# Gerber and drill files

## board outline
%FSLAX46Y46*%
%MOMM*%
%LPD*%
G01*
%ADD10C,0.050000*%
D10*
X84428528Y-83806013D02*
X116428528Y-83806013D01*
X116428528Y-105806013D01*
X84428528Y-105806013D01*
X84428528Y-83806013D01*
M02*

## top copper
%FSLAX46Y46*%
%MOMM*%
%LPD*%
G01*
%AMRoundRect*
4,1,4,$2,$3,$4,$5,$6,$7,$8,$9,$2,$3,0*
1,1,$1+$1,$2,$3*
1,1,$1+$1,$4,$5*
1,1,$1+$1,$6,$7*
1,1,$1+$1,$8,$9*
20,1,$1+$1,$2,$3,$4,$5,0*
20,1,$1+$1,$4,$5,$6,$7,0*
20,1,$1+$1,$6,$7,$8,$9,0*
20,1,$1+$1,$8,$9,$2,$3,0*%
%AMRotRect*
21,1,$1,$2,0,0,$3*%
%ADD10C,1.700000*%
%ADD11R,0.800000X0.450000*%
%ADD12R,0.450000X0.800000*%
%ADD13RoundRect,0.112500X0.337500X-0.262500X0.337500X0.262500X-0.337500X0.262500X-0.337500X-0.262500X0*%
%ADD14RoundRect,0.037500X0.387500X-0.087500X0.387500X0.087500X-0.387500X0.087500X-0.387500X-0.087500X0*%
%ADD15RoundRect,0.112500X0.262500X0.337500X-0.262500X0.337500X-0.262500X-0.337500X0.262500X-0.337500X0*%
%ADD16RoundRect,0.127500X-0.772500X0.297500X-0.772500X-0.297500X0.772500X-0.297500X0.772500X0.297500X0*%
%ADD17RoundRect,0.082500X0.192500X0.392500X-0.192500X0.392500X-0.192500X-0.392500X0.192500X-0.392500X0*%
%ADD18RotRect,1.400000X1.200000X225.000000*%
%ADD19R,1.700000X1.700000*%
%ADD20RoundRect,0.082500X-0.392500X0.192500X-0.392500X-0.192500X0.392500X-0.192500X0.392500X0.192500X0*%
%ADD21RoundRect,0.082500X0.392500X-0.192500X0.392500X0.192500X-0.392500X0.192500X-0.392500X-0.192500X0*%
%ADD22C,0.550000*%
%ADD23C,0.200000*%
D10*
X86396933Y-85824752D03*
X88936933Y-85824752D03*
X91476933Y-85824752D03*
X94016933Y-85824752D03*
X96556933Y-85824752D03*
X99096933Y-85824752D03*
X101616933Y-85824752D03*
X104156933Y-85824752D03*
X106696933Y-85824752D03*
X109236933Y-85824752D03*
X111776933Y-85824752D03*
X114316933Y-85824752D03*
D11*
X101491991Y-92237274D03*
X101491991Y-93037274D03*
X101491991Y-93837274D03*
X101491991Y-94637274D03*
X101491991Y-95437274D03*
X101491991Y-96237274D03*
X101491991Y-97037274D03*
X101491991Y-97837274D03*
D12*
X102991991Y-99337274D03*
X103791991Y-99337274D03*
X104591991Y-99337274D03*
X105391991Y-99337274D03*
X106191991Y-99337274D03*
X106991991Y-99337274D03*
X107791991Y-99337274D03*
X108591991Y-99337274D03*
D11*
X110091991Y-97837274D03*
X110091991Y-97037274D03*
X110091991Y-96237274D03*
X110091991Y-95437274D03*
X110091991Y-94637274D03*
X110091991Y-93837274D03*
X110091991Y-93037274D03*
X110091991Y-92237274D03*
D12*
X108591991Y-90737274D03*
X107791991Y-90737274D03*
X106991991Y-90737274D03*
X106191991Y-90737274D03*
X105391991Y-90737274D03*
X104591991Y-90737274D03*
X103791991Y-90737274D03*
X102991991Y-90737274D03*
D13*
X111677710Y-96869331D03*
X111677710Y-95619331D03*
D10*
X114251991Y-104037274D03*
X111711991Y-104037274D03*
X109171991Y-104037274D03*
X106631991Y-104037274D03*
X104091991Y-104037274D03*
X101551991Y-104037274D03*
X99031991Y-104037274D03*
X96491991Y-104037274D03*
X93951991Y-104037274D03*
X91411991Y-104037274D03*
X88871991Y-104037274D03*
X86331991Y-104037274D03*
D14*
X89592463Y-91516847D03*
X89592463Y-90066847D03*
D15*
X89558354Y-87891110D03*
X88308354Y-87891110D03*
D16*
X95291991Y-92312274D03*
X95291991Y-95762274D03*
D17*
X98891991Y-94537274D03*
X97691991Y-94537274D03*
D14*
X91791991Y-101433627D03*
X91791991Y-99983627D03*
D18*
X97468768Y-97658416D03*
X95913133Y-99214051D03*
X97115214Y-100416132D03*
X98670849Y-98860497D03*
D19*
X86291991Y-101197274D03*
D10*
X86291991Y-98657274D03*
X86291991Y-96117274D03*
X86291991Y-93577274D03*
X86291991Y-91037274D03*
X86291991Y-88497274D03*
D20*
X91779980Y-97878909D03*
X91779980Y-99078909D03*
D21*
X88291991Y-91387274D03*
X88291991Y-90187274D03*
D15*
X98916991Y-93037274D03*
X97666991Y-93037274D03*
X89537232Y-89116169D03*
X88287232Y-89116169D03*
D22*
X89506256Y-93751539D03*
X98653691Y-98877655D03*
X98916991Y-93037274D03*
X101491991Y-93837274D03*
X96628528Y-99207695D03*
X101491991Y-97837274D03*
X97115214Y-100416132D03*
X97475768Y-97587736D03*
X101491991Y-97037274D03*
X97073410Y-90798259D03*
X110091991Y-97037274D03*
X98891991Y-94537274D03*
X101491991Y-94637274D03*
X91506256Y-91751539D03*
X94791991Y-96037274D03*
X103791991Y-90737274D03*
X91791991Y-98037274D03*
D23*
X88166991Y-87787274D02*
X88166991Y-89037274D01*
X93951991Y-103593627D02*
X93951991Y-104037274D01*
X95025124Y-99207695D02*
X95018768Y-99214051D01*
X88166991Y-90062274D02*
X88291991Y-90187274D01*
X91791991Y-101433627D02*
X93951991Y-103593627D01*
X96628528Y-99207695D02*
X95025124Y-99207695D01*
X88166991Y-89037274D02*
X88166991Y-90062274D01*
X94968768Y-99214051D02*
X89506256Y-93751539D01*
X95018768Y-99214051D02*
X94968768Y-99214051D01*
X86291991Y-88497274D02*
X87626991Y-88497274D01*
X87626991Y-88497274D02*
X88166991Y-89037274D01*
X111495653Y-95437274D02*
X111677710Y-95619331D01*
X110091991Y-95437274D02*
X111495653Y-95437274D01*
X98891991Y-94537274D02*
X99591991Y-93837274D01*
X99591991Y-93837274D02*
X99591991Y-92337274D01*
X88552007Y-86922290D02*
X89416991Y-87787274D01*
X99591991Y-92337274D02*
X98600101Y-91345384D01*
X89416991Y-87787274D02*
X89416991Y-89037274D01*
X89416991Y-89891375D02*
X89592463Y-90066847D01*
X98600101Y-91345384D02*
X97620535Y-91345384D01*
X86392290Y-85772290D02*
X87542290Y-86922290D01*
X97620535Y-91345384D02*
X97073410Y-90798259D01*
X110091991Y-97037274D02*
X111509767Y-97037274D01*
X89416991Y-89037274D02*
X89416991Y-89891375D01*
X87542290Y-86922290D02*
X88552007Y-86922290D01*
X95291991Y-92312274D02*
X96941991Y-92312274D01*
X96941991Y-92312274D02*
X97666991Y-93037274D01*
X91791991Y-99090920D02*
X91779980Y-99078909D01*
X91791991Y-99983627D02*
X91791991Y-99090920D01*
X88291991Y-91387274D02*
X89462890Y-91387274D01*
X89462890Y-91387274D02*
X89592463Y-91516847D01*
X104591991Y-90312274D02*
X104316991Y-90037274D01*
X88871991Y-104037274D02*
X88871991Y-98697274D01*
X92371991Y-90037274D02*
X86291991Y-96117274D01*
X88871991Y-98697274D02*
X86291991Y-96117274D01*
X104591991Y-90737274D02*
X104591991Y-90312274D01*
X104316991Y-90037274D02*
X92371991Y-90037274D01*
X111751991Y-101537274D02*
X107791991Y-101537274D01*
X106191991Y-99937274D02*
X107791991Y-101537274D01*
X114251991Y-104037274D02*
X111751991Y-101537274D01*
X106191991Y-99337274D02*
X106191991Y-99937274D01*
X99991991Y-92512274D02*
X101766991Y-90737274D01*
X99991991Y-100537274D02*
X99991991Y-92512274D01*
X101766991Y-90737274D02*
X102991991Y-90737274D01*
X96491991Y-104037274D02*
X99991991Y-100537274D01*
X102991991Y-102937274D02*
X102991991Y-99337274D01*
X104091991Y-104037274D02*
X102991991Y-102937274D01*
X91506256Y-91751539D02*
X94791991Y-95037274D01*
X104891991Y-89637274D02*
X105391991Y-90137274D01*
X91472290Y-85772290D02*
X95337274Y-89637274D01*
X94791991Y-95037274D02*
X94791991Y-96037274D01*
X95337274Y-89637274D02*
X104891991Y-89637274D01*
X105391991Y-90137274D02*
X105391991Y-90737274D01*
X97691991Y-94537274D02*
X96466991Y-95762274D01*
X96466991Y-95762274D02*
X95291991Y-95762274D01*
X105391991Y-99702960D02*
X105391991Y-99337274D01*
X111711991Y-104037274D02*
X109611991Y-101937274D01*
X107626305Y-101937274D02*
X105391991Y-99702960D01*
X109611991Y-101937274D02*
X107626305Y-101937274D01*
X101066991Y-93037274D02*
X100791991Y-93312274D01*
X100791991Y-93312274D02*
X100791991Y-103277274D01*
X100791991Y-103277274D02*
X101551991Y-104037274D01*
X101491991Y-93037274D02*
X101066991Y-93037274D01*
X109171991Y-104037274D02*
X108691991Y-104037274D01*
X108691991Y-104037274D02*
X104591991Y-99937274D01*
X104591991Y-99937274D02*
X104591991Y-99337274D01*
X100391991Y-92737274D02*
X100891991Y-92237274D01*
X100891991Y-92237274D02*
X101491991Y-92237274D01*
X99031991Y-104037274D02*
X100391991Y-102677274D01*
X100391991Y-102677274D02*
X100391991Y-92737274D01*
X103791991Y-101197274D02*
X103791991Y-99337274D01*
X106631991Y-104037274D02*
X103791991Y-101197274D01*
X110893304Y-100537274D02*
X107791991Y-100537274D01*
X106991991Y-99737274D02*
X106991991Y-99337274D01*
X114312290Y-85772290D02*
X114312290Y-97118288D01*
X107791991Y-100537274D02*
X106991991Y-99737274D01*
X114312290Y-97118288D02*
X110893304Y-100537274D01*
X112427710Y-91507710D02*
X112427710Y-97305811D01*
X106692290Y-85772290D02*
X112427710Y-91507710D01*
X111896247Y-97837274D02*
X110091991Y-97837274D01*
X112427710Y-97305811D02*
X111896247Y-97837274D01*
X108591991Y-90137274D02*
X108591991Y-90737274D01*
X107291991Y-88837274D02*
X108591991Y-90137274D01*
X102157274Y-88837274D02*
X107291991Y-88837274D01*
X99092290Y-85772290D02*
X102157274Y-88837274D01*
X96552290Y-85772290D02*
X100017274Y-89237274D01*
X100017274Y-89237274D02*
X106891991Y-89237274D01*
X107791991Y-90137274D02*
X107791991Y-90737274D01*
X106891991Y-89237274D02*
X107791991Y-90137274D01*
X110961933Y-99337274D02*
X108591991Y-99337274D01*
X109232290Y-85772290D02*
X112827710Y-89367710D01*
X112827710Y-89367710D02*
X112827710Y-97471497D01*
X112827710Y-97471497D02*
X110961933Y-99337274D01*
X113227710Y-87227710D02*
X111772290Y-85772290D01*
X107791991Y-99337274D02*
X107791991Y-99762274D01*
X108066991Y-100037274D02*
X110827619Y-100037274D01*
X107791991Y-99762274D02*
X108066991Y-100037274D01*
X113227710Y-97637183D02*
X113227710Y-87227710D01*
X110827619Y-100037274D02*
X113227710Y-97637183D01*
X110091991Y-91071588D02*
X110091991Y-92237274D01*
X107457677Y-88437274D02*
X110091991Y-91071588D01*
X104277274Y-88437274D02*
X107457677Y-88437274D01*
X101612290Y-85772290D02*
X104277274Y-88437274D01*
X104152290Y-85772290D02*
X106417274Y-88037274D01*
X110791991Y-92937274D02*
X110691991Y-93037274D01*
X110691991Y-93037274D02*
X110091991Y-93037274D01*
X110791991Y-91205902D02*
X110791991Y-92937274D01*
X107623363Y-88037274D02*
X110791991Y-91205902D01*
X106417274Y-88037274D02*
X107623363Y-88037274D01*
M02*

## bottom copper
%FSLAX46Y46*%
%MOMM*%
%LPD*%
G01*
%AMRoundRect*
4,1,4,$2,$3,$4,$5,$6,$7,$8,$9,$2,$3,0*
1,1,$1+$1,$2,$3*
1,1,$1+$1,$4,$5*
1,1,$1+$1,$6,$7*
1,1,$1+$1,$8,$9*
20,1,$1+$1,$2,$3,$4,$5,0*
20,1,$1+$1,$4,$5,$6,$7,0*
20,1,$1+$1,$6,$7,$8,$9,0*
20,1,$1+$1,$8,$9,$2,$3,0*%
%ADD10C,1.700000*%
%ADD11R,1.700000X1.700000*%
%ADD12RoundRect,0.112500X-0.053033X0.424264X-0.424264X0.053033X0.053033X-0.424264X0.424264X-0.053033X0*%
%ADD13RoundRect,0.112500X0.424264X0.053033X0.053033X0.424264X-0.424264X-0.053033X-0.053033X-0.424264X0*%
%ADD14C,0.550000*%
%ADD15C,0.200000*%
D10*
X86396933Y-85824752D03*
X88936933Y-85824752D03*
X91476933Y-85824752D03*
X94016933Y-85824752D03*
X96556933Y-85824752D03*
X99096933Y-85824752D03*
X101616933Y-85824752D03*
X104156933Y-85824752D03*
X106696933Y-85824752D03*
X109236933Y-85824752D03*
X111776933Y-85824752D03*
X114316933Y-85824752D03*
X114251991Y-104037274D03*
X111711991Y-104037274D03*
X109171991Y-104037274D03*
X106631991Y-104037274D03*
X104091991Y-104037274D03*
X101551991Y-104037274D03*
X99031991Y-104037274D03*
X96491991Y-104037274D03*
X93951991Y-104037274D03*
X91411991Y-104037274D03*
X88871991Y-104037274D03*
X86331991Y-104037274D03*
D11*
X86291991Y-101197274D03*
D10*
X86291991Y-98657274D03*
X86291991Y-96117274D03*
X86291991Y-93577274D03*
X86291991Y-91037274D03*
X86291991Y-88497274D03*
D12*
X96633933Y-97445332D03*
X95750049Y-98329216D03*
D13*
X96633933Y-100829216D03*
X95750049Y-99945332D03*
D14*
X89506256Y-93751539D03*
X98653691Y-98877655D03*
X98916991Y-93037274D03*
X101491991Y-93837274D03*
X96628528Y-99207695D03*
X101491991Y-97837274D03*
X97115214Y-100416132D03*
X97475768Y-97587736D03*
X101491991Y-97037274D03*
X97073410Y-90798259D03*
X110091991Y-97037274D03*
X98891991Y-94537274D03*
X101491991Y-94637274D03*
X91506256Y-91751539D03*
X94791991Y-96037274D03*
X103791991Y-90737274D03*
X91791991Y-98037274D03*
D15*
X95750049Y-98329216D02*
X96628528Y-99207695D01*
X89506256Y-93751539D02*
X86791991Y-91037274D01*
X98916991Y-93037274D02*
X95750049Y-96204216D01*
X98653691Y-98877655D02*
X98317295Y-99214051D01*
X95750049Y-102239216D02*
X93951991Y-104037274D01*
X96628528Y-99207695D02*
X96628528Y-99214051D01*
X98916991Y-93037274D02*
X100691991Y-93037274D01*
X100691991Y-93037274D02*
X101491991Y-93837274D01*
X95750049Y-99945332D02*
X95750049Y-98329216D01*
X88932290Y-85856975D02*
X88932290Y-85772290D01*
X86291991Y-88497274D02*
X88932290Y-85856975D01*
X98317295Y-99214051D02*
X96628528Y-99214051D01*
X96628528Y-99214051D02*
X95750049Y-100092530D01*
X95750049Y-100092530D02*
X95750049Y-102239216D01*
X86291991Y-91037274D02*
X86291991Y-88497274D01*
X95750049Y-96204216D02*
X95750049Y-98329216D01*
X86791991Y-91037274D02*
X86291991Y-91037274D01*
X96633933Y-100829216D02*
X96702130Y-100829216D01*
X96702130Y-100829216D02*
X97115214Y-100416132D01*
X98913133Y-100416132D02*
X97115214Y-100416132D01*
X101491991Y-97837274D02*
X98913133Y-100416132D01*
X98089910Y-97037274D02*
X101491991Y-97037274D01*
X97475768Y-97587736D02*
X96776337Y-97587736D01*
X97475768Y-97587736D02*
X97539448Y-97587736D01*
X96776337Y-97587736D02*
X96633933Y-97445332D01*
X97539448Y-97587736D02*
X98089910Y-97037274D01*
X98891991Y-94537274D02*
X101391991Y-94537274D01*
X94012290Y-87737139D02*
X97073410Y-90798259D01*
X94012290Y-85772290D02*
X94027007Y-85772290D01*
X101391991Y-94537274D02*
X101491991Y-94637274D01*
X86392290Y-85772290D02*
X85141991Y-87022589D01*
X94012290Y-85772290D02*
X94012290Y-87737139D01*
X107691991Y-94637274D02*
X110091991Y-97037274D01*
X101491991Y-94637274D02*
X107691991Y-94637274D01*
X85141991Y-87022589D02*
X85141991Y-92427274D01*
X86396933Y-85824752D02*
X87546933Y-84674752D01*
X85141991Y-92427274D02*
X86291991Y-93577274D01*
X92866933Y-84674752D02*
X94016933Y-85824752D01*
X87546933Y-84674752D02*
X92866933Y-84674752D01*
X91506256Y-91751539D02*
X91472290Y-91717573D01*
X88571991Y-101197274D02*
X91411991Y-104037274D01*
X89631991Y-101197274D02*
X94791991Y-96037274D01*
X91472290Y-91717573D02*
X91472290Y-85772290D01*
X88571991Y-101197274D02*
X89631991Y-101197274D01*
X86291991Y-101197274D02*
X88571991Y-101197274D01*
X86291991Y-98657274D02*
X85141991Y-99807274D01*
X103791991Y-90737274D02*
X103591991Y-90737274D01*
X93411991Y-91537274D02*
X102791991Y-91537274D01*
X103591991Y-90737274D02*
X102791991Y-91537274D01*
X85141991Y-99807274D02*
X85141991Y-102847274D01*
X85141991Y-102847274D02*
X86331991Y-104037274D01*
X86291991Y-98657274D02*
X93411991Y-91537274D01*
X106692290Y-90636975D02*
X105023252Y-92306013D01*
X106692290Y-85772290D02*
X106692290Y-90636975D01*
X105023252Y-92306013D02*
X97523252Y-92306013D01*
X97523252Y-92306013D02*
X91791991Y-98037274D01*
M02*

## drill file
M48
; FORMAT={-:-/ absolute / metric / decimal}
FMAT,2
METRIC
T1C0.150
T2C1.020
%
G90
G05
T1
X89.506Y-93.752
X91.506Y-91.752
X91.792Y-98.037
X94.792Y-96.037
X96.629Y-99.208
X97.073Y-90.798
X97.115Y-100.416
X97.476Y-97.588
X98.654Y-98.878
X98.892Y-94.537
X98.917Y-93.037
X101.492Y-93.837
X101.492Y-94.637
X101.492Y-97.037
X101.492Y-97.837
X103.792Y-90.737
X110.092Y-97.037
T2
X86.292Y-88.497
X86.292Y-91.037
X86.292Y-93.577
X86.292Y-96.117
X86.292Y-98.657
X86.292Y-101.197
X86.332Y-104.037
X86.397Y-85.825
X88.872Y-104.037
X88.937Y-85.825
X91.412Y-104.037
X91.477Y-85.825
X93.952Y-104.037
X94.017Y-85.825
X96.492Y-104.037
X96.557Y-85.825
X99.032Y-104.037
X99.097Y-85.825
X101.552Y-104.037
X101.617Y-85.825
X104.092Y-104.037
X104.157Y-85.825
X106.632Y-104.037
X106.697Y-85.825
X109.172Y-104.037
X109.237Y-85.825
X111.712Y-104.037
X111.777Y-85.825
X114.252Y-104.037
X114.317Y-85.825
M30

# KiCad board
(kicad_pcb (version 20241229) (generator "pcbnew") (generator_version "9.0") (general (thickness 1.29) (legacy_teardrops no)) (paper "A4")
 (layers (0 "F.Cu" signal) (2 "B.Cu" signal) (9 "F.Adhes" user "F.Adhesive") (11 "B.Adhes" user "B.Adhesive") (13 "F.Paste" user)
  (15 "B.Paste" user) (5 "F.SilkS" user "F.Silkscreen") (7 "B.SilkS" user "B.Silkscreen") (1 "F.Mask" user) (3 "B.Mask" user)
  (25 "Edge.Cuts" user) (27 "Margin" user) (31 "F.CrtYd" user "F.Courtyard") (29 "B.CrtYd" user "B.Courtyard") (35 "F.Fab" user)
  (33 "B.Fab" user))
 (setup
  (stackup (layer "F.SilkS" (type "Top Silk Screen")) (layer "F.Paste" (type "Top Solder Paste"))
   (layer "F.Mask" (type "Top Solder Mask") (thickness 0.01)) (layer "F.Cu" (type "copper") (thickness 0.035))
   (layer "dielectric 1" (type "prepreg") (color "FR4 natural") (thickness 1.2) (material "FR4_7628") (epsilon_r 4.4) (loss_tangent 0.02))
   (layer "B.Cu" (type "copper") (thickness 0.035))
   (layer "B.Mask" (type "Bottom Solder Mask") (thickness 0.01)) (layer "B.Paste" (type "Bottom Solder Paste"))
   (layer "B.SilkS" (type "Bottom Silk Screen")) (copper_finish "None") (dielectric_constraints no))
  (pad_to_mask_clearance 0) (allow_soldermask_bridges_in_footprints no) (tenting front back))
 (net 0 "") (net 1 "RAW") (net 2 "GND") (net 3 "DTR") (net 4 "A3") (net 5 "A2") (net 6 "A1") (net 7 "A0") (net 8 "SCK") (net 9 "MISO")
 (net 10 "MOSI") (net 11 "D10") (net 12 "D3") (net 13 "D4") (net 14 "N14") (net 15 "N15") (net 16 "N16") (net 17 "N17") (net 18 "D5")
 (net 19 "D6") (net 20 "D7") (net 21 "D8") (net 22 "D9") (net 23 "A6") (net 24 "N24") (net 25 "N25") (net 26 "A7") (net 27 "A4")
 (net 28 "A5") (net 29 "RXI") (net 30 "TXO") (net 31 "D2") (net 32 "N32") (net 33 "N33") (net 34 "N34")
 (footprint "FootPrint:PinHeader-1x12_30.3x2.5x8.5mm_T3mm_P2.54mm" (layer "F.Cu") (at 100.356933 85.824752)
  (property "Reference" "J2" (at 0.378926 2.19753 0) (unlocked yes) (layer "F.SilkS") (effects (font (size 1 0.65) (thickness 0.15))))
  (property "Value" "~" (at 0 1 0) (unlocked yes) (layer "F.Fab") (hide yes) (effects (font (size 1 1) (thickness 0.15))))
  (pad "1" thru_hole circle (at -13.96 0) (size 1.7 1.7) (drill 1.02) (layers "*.Cu" "*.Mask") (remove_unused_layers no) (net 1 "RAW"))
  (pad "2" thru_hole circle (at -11.42 0) (size 1.7 1.7) (drill 1.02) (layers "*.Cu" "*.Mask") (remove_unused_layers no) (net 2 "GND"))
  (pad "3" thru_hole circle (at -8.88 0) (size 1.7 1.7) (drill 1.02) (layers "*.Cu" "*.Mask") (remove_unused_layers no) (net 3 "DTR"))
  (pad "4" thru_hole circle (at -6.34 0) (size 1.7 1.7) (drill 1.02) (layers "*.Cu" "*.Mask") (remove_unused_layers no) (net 1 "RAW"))
  (pad "5" thru_hole circle (at -3.8 0) (size 1.7 1.7) (drill 1.02) (layers "*.Cu" "*.Mask") (remove_unused_layers no) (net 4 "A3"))
  (pad "6" thru_hole circle (at -1.26 0) (size 1.7 1.7) (drill 1.02) (layers "*.Cu" "*.Mask") (remove_unused_layers no) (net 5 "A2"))
  (pad "7" thru_hole circle (at 1.26 0) (size 1.7 1.7) (drill 1.02) (layers "*.Cu" "*.Mask") (remove_unused_layers no) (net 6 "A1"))
  (pad "8" thru_hole circle (at 3.8 0) (size 1.7 1.7) (drill 1.02) (layers "*.Cu" "*.Mask") (remove_unused_layers no) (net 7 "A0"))
  (pad "9" thru_hole circle (at 6.34 0) (size 1.7 1.7) (drill 1.02) (layers "*.Cu" "*.Mask") (remove_unused_layers no) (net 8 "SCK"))
  (pad "10" thru_hole circle (at 8.88 0) (size 1.7 1.7) (drill 1.02) (layers "*.Cu" "*.Mask") (remove_unused_layers no) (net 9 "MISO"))
  (pad "11" thru_hole circle (at 11.42 0) (size 1.7 1.7) (drill 1.02) (layers "*.Cu" "*.Mask") (remove_unused_layers no) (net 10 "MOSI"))
  (pad "12" thru_hole circle (at 13.96 0) (size 1.7 1.7) (drill 1.02) (layers "*.Cu" "*.Mask") (remove_unused_layers no) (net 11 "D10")))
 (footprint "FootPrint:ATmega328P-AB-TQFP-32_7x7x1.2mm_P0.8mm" (layer "F.Cu") (at 105.791991 95.037274)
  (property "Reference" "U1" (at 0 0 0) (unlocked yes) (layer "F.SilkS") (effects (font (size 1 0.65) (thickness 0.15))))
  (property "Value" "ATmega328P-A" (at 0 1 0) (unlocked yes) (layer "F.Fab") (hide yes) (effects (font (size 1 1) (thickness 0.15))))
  (pad "1" smd rect (at -4.3 -2.8) (size 0.8 0.45) (layers "F.Cu" "F.Mask" "F.Paste") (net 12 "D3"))
  (pad "2" smd rect (at -4.3 -2) (size 0.8 0.45) (layers "F.Cu" "F.Mask" "F.Paste") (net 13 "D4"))
  (pad "3" smd rect (at -4.3 -1.2) (size 0.8 0.45) (layers "F.Cu" "F.Mask" "F.Paste") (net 2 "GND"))
  (pad "4" smd rect (at -4.3 -0.4) (size 0.8 0.45) (layers "F.Cu" "F.Mask" "F.Paste") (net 1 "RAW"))
  (pad "5" smd rect (at -4.3 0.4) (size 0.8 0.45) (layers "F.Cu" "F.Mask" "F.Paste") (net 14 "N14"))
  (pad "6" smd rect (at -4.3 1.2) (size 0.8 0.45) (layers "F.Cu" "F.Mask" "F.Paste") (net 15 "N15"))
  (pad "7" smd rect (at -4.3 2) (size 0.8 0.45) (layers "F.Cu" "F.Mask" "F.Paste") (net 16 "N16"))
  (pad "8" smd rect (at -4.3 2.8) (size 0.8 0.45) (layers "F.Cu" "F.Mask" "F.Paste") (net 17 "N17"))
  (pad "9" smd rect (at -2.8 4.3 90) (size 0.8 0.45) (layers "F.Cu" "F.Mask" "F.Paste") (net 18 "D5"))
  (pad "10" smd rect (at -2 4.3 90) (size 0.8 0.45) (layers "F.Cu" "F.Mask" "F.Paste") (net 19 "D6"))
  (pad "11" smd rect (at -1.2 4.3 90) (size 0.8 0.45) (layers "F.Cu" "F.Mask" "F.Paste") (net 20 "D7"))
  (pad "12" smd rect (at -0.4 4.3 90) (size 0.8 0.45) (layers "F.Cu" "F.Mask" "F.Paste") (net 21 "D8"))
  (pad "13" smd rect (at 0.4 4.3 90) (size 0.8 0.45) (layers "F.Cu" "F.Mask" "F.Paste") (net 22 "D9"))
  (pad "14" smd rect (at 1.2 4.3 90) (size 0.8 0.45) (layers "F.Cu" "F.Mask" "F.Paste") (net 11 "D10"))
  (pad "15" smd rect (at 2 4.3 90) (size 0.8 0.45) (layers "F.Cu" "F.Mask" "F.Paste") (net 10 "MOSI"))
  (pad "16" smd rect (at 2.8 4.3 90) (size 0.8 0.45) (layers "F.Cu" "F.Mask" "F.Paste") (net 9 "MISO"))
  (pad "17" smd rect (at 4.3 2.8) (size 0.8 0.45) (layers "F.Cu" "F.Mask" "F.Paste") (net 8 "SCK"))
  (pad "18" smd rect (at 4.3 2) (size 0.8 0.45) (layers "F.Cu" "F.Mask" "F.Paste") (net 1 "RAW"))
  (pad "19" smd rect (at 4.3 1.2) (size 0.8 0.45) (layers "F.Cu" "F.Mask" "F.Paste") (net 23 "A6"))
  (pad "20" smd rect (at 4.3 0.4) (size 0.8 0.45) (layers "F.Cu" "F.Mask" "F.Paste") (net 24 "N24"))
  (pad "21" smd rect (at 4.3 -0.4) (size 0.8 0.45) (layers "F.Cu" "F.Mask" "F.Paste") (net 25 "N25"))
  (pad "22" smd rect (at 4.3 -1.2) (size 0.8 0.45) (layers "F.Cu" "F.Mask" "F.Paste") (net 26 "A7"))
  (pad "23" smd rect (at 4.3 -2) (size 0.8 0.45) (layers "F.Cu" "F.Mask" "F.Paste") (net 7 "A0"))
  (pad "24" smd rect (at 4.3 -2.8) (size 0.8 0.45) (layers "F.Cu" "F.Mask" "F.Paste") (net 6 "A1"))
  (pad "25" smd rect (at 2.8 -4.3 90) (size 0.8 0.45) (layers "F.Cu" "F.Mask" "F.Paste") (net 5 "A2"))
  (pad "26" smd rect (at 2 -4.3 90) (size 0.8 0.45) (layers "F.Cu" "F.Mask" "F.Paste") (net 4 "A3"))
  (pad "27" smd rect (at 1.2 -4.3 90) (size 0.8 0.45) (layers "F.Cu" "F.Mask" "F.Paste") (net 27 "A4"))
  (pad "28" smd rect (at 0.4 -4.3 90) (size 0.8 0.45) (layers "F.Cu" "F.Mask" "F.Paste") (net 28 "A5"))
  (pad "29" smd rect (at -0.4 -4.3 90) (size 0.8 0.45) (layers "F.Cu" "F.Mask" "F.Paste") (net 3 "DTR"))
  (pad "30" smd rect (at -1.2 -4.3 90) (size 0.8 0.45) (layers "F.Cu" "F.Mask" "F.Paste") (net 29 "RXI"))
  (pad "31" smd rect (at -2 -4.3 90) (size 0.8 0.45) (layers "F.Cu" "F.Mask" "F.Paste") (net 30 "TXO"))
  (pad "32" smd rect (at -2.8 -4.3 90) (size 0.8 0.45) (layers "F.Cu" "F.Mask" "F.Paste") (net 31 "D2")))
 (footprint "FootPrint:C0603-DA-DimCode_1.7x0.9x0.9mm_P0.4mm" (layer "F.Cu") (at 111.67771 96.244331 90)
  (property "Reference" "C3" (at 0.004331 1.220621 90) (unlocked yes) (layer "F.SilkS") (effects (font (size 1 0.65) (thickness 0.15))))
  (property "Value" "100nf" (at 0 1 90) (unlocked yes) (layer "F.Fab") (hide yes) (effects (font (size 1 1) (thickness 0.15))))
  (pad "1" smd roundrect (at -0.625 0 90) (size 0.75 0.9) (layers "F.Cu" "F.Mask" "F.Paste") (roundrect_rratio 0.15) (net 1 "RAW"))
  (pad "2" smd roundrect (at 0.625 0 90) (size 0.75 0.9) (layers "F.Cu" "F.Mask" "F.Paste") (roundrect_rratio 0.15) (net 24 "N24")))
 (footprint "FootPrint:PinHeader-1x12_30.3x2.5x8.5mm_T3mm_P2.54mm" (layer "F.Cu") (at 100.291991 104.037274 180)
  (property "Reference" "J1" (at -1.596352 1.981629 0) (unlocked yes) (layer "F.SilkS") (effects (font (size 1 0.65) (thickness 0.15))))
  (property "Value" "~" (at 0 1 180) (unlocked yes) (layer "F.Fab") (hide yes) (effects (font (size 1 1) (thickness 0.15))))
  (pad "1" thru_hole circle (at -13.96 0 180) (size 1.7 1.7) (drill 1.02) (layers "*.Cu" "*.Mask") (remove_unused_layers no) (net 22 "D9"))
  (pad "2" thru_hole circle (at -11.42 0 180) (size 1.7 1.7) (drill 1.02) (layers "*.Cu" "*.Mask") (remove_unused_layers no) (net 21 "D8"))
  (pad "3" thru_hole circle (at -8.88 0 180) (size 1.7 1.7) (drill 1.02) (layers "*.Cu" "*.Mask") (remove_unused_layers no) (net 20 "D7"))
  (pad "4" thru_hole circle (at -6.34 0 180) (size 1.7 1.7) (drill 1.02) (layers "*.Cu" "*.Mask") (remove_unused_layers no) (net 19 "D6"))
  (pad "5" thru_hole circle (at -3.8 0 180) (size 1.7 1.7) (drill 1.02) (layers "*.Cu" "*.Mask") (remove_unused_layers no) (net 18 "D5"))
  (pad "6" thru_hole circle (at -1.26 0 180) (size 1.7 1.7) (drill 1.02) (layers "*.Cu" "*.Mask") (remove_unused_layers no) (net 13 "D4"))
  (pad "7" thru_hole circle (at 1.26 0 180) (size 1.7 1.7) (drill 1.02) (layers "*.Cu" "*.Mask") (remove_unused_layers no) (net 12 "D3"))
  (pad "8" thru_hole circle (at 3.8 0 180) (size 1.7 1.7) (drill 1.02) (layers "*.Cu" "*.Mask") (remove_unused_layers no) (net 31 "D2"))
  (pad "9" thru_hole circle (at 6.34 0 180) (size 1.7 1.7) (drill 1.02) (layers "*.Cu" "*.Mask") (remove_unused_layers no) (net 2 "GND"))
  (pad "10" thru_hole circle (at 8.88 0 180) (size 1.7 1.7) (drill 1.02) (layers "*.Cu" "*.Mask") (remove_unused_layers no) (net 3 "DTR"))
  (pad "11" thru_hole circle (at 11.42 0 180) (size 1.7 1.7) (drill 1.02) (layers "*.Cu" "*.Mask") (remove_unused_layers no) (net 29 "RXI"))
  (pad "12" thru_hole circle (at 13.96 0 180) (size 1.7 1.7) (drill 1.02) (layers "*.Cu" "*.Mask") (remove_unused_layers no) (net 30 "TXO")))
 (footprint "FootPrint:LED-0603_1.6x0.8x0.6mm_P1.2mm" (layer "F.Cu") (at 89.592463 90.791847 90)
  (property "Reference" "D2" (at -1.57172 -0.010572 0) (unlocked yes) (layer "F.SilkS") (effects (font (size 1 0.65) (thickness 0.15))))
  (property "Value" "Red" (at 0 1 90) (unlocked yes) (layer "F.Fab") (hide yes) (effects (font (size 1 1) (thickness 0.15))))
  (pad "1" smd roundrect (at -0.725 0 90) (size 0.25 0.85) (layers "F.Cu" "F.Mask" "F.Paste") (roundrect_rratio 0.15) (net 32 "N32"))
  (pad "2" smd roundrect (at 0.725 0 90) (size 0.25 0.85) (layers "F.Cu" "F.Mask" "F.Paste") (roundrect_rratio 0.15) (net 1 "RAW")))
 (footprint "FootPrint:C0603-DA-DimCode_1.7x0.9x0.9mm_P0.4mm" (layer "F.Cu") (at 88.933354 87.89111 180)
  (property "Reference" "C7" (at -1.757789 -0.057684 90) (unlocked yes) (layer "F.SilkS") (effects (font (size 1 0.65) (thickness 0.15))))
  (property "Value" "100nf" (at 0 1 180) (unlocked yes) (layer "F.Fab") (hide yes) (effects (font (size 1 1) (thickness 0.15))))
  (pad "1" smd roundrect (at -0.625 0 180) (size 0.75 0.9) (layers "F.Cu" "F.Mask" "F.Paste") (roundrect_rratio 0.15) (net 1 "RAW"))
  (pad "2" smd roundrect (at 0.625 0 180) (size 0.75 0.9) (layers "F.Cu" "F.Mask" "F.Paste") (roundrect_rratio 0.15) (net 2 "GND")))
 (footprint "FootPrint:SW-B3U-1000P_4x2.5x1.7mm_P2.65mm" (layer "F.Cu") (at 95.291991 94.037274 -90)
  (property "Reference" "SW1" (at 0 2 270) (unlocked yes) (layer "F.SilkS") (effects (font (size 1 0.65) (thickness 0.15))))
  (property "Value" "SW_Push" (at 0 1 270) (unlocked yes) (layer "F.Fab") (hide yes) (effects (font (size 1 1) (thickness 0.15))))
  (pad "1" smd roundrect (at -1.725 0 270) (size 0.85 1.8) (layers "F.Cu" "F.Mask" "F.Paste") (roundrect_rratio 0.15) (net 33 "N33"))
  (pad "2" smd roundrect (at 1.725 0 270) (size 0.85 1.8) (layers "F.Cu" "F.Mask" "F.Paste") (roundrect_rratio 0.15) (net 3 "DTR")))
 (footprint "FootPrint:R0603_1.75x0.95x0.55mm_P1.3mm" (layer "F.Cu") (at 98.291991 94.537274 180)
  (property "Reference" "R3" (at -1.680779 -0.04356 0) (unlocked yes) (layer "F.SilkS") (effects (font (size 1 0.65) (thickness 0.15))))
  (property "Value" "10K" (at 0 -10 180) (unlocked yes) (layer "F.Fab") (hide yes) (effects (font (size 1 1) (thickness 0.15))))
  (pad "1" smd roundrect (at -0.6 0 180) (size 0.55 0.95) (layers "F.Cu" "F.Mask" "F.Paste") (roundrect_rratio 0.15) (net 1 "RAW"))
  (pad "2" smd roundrect (at 0.6 0 180) (size 0.55 0.95) (layers "F.Cu" "F.Mask" "F.Paste") (roundrect_rratio 0.15) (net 3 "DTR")))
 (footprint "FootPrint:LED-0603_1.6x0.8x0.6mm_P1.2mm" (layer "F.Cu") (at 91.791991 100.708627 90)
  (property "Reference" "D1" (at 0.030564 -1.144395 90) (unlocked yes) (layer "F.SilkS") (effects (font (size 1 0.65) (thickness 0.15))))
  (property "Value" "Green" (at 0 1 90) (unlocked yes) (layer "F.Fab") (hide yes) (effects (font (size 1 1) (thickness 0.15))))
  (pad "1" smd roundrect (at -0.725 0 90) (size 0.25 0.85) (layers "F.Cu" "F.Mask" "F.Paste") (roundrect_rratio 0.15) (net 2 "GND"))
  (pad "2" smd roundrect (at 0.725 0 90) (size 0.25 0.85) (layers "F.Cu" "F.Mask" "F.Paste") (roundrect_rratio 0.15) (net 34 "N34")))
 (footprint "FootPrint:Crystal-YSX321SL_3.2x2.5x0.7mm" (layer "F.Cu") (at 97.291991 99.037274 -135)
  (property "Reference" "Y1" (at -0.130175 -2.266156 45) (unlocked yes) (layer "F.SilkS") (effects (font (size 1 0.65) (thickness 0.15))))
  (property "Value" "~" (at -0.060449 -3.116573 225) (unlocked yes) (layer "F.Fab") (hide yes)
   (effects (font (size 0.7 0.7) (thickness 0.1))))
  (pad "1" smd rect (at -1.1 0.85 225) (size 1.4 1.2) (layers "F.Cu" "F.Mask" "F.Paste") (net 16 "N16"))
  (pad "2" smd rect (at 1.1 0.85 225) (size 1.4 1.2) (layers "F.Cu" "F.Mask" "F.Paste") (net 2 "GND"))
  (pad "3" smd rect (at 1.1 -0.85 225) (size 1.4 1.2) (layers "F.Cu" "F.Mask" "F.Paste") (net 17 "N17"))
  (pad "4" smd rect (at -1.1 -0.85 225) (size 1.4 1.2) (layers "F.Cu" "F.Mask" "F.Paste") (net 2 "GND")))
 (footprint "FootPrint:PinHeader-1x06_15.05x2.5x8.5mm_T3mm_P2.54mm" (layer "F.Cu") (at 86.291991 94.847274 90)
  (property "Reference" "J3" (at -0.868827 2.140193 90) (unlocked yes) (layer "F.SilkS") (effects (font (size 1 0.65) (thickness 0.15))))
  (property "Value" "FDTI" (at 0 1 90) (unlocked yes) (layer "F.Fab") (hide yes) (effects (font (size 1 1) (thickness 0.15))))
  (pad "1" thru_hole rect (at -6.35 0 90) (size 1.7 1.7) (drill 1.02) (layers "*.Cu" "*.Mask") (remove_unused_layers no) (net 3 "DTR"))
  (pad "2" thru_hole circle (at -3.81 0 90) (size 1.7 1.7) (drill 1.02) (layers "*.Cu" "*.Mask") (remove_unused_layers no) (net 30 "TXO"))
  (pad "3" thru_hole circle (at -1.27 0 90) (size 1.7 1.7) (drill 1.02) (layers "*.Cu" "*.Mask") (remove_unused_layers no) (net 29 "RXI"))
  (pad "4" thru_hole circle (at 1.27 0 90) (size 1.7 1.7) (drill 1.02) (layers "*.Cu" "*.Mask") (remove_unused_layers no) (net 1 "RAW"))
  (pad "5" thru_hole circle (at 3.81 0 90) (size 1.7 1.7) (drill 1.02) (layers "*.Cu" "*.Mask") (remove_unused_layers no) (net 2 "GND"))
  (pad "6" thru_hole circle (at 6.35 0 90) (size 1.7 1.7) (drill 1.02) (layers "*.Cu" "*.Mask") (remove_unused_layers no) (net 2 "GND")))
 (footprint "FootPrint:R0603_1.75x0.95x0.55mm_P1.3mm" (layer "F.Cu") (at 91.77998 98.478909 -90)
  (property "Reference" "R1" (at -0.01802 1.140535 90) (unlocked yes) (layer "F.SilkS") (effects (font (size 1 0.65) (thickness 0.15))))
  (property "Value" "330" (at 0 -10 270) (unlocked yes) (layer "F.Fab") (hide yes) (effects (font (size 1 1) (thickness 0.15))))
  (pad "1" smd roundrect (at -0.6 0 270) (size 0.55 0.95) (layers "F.Cu" "F.Mask" "F.Paste") (roundrect_rratio 0.15) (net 8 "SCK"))
  (pad "2" smd roundrect (at 0.6 0 270) (size 0.55 0.95) (layers "F.Cu" "F.Mask" "F.Paste") (roundrect_rratio 0.15) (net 34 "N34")))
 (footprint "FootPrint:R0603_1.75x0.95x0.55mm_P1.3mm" (layer "F.Cu") (at 88.291991 90.787274 90)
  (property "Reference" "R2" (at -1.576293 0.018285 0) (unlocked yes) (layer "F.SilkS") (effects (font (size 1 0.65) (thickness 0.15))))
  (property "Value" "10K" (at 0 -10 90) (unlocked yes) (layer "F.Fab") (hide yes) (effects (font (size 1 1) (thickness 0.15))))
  (pad "1" smd roundrect (at -0.6 0 90) (size 0.55 0.95) (layers "F.Cu" "F.Mask" "F.Paste") (roundrect_rratio 0.15) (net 32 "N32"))
  (pad "2" smd roundrect (at 0.6 0 90) (size 0.55 0.95) (layers "F.Cu" "F.Mask" "F.Paste") (roundrect_rratio 0.15) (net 2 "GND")))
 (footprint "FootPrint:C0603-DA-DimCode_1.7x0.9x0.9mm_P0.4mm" (layer "F.Cu") (at 98.291991 93.037274 180)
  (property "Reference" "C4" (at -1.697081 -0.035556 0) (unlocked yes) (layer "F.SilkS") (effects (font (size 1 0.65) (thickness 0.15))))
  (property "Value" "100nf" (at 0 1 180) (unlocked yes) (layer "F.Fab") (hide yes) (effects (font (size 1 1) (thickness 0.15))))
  (pad "1" smd roundrect (at -0.625 0 180) (size 0.75 0.9) (layers "F.Cu" "F.Mask" "F.Paste") (roundrect_rratio 0.15) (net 2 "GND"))
  (pad "2" smd roundrect (at 0.625 0 180) (size 0.75 0.9) (layers "F.Cu" "F.Mask" "F.Paste") (roundrect_rratio 0.15) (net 33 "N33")))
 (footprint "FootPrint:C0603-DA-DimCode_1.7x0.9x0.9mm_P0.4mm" (layer "F.Cu") (at 88.912232 89.116169 180)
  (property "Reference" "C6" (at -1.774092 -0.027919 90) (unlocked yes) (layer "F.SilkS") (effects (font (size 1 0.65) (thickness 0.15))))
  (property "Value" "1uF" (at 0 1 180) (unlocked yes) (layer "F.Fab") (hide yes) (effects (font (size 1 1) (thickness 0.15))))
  (pad "1" smd roundrect (at -0.625 0 180) (size 0.75 0.9) (layers "F.Cu" "F.Mask" "F.Paste") (roundrect_rratio 0.15) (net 1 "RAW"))
  (pad "2" smd roundrect (at 0.625 0 180) (size 0.75 0.9) (layers "F.Cu" "F.Mask" "F.Paste") (roundrect_rratio 0.15) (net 2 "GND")))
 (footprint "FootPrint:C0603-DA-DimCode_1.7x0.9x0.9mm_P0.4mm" (layer "B.Cu") (at 96.191991 97.887274 -135)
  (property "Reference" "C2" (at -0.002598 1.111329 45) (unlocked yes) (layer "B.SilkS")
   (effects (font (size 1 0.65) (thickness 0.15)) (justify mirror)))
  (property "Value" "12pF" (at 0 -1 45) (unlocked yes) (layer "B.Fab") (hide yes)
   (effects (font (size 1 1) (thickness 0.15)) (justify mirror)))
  (pad "1" smd roundrect (at -0.625 0 225) (size 0.75 0.9) (layers "B.Cu" "B.Mask" "B.Paste") (roundrect_rratio 0.15) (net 16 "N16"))
  (pad "2" smd roundrect (at 0.625 0 225) (size 0.75 0.9) (layers "B.Cu" "B.Mask" "B.Paste") (roundrect_rratio 0.15) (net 2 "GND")))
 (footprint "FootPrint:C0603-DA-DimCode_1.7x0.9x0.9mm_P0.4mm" (layer "B.Cu") (at 96.191991 100.387274 135)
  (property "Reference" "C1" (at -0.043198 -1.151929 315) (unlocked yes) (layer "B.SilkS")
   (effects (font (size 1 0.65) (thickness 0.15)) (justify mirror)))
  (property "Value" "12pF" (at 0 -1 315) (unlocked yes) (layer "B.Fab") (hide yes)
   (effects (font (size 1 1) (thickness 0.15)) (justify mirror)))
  (pad "1" smd roundrect (at -0.625 0 135) (size 0.75 0.9) (layers "B.Cu" "B.Mask" "B.Paste") (roundrect_rratio 0.15) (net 17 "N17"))
  (pad "2" smd roundrect (at 0.625 0 135) (size 0.75 0.9) (layers "B.Cu" "B.Mask" "B.Paste") (roundrect_rratio 0.15) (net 2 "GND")))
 (gr_rect (start 84.428528 83.806013) (end 116.428528 105.806013) (stroke (width 0.05) (type solid)) (fill no) (layer "Edge.Cuts"))
 (segment (start 88.166991 87.787274) (end 88.166991 89.037274) (width 0.2) (layer "F.Cu") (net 2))
 (segment (start 93.951991 103.593627) (end 93.951991 104.037274) (width 0.2) (layer "F.Cu") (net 2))
 (segment (start 95.025124 99.207695) (end 95.018768 99.214051) (width 0.2) (layer "F.Cu") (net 2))
 (segment (start 88.166991 90.062274) (end 88.291991 90.187274) (width 0.2) (layer "F.Cu") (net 2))
 (segment (start 91.791991 101.433627) (end 93.951991 103.593627) (width 0.2) (layer "F.Cu") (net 2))
 (segment (start 96.628528 99.207695) (end 95.025124 99.207695) (width 0.2) (layer "F.Cu") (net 2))
 (segment (start 88.166991 89.037274) (end 88.166991 90.062274) (width 0.2) (layer "F.Cu") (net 2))
 (segment (start 94.968768 99.214051) (end 89.506256 93.751539) (width 0.2) (layer "F.Cu") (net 2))
 (segment (start 95.018768 99.214051) (end 94.968768 99.214051) (width 0.2) (layer "F.Cu") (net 2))
 (segment (start 86.291991 88.497274) (end 87.626991 88.497274) (width 0.2) (layer "F.Cu") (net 2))
 (segment (start 87.626991 88.497274) (end 88.166991 89.037274) (width 0.2) (layer "F.Cu") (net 2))
 (via (at 89.506256 93.751539) (size 0.55) (drill 0.15) (layers "F.Cu" "B.Cu") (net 2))
 (via (at 98.653691 98.877655) (size 0.55) (drill 0.15) (layers "F.Cu" "B.Cu") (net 2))
 (via (at 98.916991 93.037274) (size 0.55) (drill 0.15) (layers "F.Cu" "B.Cu") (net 2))
 (via (at 101.491991 93.837274) (size 0.55) (drill 0.15) (layers "F.Cu" "B.Cu") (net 2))
 (via (at 96.628528 99.207695) (size 0.55) (drill 0.15) (layers "F.Cu" "B.Cu") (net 2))
 (segment (start 95.750049 98.329216) (end 96.628528 99.207695) (width 0.2) (layer "B.Cu") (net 2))
 (segment (start 89.506256 93.751539) (end 86.791991 91.037274) (width 0.2) (layer "B.Cu") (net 2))
 (segment (start 98.916991 93.037274) (end 95.750049 96.204216) (width 0.2) (layer "B.Cu") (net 2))
 (segment (start 98.653691 98.877655) (end 98.317295 99.214051) (width 0.2) (layer "B.Cu") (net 2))
 (segment (start 95.750049 102.239216) (end 93.951991 104.037274) (width 0.2) (layer "B.Cu") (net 2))
 (segment (start 96.628528 99.207695) (end 96.628528 99.214051) (width 0.2) (layer "B.Cu") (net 2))
 (segment (start 98.916991 93.037274) (end 100.691991 93.037274) (width 0.2) (layer "B.Cu") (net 2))
 (segment (start 100.691991 93.037274) (end 101.491991 93.837274) (width 0.2) (layer "B.Cu") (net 2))
 (segment (start 95.750049 99.945332) (end 95.750049 98.329216) (width 0.2) (layer "B.Cu") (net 2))
 (segment (start 88.93229 85.856975) (end 88.93229 85.77229) (width 0.2) (layer "B.Cu") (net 2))
 (segment (start 86.291991 88.497274) (end 88.93229 85.856975) (width 0.2) (layer "B.Cu") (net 2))
 (segment (start 98.317295 99.214051) (end 96.628528 99.214051) (width 0.2) (layer "B.Cu") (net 2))
 (segment (start 96.628528 99.214051) (end 95.750049 100.09253) (width 0.2) (layer "B.Cu") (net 2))
 (segment (start 95.750049 100.09253) (end 95.750049 102.239216) (width 0.2) (layer "B.Cu") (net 2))
 (segment (start 86.291991 91.037274) (end 86.291991 88.497274) (width 0.2) (layer "B.Cu") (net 2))
 (segment (start 95.750049 96.204216) (end 95.750049 98.329216) (width 0.2) (layer "B.Cu") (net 2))
 (segment (start 86.791991 91.037274) (end 86.291991 91.037274) (width 0.2) (layer "B.Cu") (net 2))
 (via (at 101.491991 97.837274) (size 0.55) (drill 0.15) (layers "F.Cu" "B.Cu") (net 17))
 (via (at 97.115214 100.416132) (size 0.55) (drill 0.15) (layers "F.Cu" "B.Cu") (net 17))
 (segment (start 96.633933 100.829216) (end 96.70213 100.829216) (width 0.2) (layer "B.Cu") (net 17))
 (segment (start 96.70213 100.829216) (end 97.115214 100.416132) (width 0.2) (layer "B.Cu") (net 17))
 (segment (start 98.913133 100.416132) (end 97.115214 100.416132) (width 0.2) (layer "B.Cu") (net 17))
 (segment (start 101.491991 97.837274) (end 98.913133 100.416132) (width 0.2) (layer "B.Cu") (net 17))
 (via (at 97.475768 97.587736) (size 0.55) (drill 0.15) (layers "F.Cu" "B.Cu") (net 16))
 (via (at 101.491991 97.037274) (size 0.55) (drill 0.15) (layers "F.Cu" "B.Cu") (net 16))
 (segment (start 98.08991 97.037274) (end 101.491991 97.037274) (width 0.2) (layer "B.Cu") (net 16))
 (segment (start 97.475768 97.587736) (end 96.776337 97.587736) (width 0.2) (layer "B.Cu") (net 16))
 (segment (start 97.475768 97.587736) (end 97.539448 97.587736) (width 0.2) (layer "B.Cu") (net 16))
 (segment (start 96.776337 97.587736) (end 96.633933 97.445332) (width 0.2) (layer "B.Cu") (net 16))
 (segment (start 97.539448 97.587736) (end 98.08991 97.037274) (width 0.2) (layer "B.Cu") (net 16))
 (segment (start 111.495653 95.437274) (end 111.67771 95.619331) (width 0.2) (layer "F.Cu") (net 24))
 (segment (start 110.091991 95.437274) (end 111.495653 95.437274) (width 0.2) (layer "F.Cu") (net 24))
 (segment (start 98.891991 94.537274) (end 99.591991 93.837274) (width 0.2) (layer "F.Cu") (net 1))
 (segment (start 99.591991 93.837274) (end 99.591991 92.337274) (width 0.2) (layer "F.Cu") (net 1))
 (segment (start 88.552007 86.92229) (end 89.416991 87.787274) (width 0.2) (layer "F.Cu") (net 1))
 (segment (start 99.591991 92.337274) (end 98.600101 91.345384) (width 0.2) (layer "F.Cu") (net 1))
 (segment (start 89.416991 87.787274) (end 89.416991 89.037274) (width 0.2) (layer "F.Cu") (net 1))
 (segment (start 89.416991 89.891375) (end 89.592463 90.066847) (width 0.2) (layer "F.Cu") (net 1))
 (segment (start 98.600101 91.345384) (end 97.620535 91.345384) (width 0.2) (layer "F.Cu") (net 1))
 (segment (start 86.39229 85.77229) (end 87.54229 86.92229) (width 0.2) (layer "F.Cu") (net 1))
 (segment (start 97.620535 91.345384) (end 97.07341 90.798259) (width 0.2) (layer "F.Cu") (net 1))
 (segment (start 110.091991 97.037274) (end 111.509767 97.037274) (width 0.2) (layer "F.Cu") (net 1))
 (segment (start 89.416991 89.037274) (end 89.416991 89.891375) (width 0.2) (layer "F.Cu") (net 1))
 (segment (start 87.54229 86.92229) (end 88.552007 86.92229) (width 0.2) (layer "F.Cu") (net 1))
 (via (at 97.07341 90.798259) (size 0.55) (drill 0.15) (layers "F.Cu" "B.Cu") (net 1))
 (via (at 110.091991 97.037274) (size 0.55) (drill 0.15) (layers "F.Cu" "B.Cu") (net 1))
 (via (at 98.891991 94.537274) (size 0.55) (drill 0.15) (layers "F.Cu" "B.Cu") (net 1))
 (via (at 101.491991 94.637274) (size 0.55) (drill 0.15) (layers "F.Cu" "B.Cu") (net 1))
 (segment (start 98.891991 94.537274) (end 101.391991 94.537274) (width 0.2) (layer "B.Cu") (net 1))
 (segment (start 94.01229 87.737139) (end 97.07341 90.798259) (width 0.2) (layer "B.Cu") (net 1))
 (segment (start 94.01229 85.77229) (end 94.027007 85.77229) (width 0.2) (layer "B.Cu") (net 1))
 (segment (start 101.391991 94.537274) (end 101.491991 94.637274) (width 0.2) (layer "B.Cu") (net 1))
 (segment (start 86.39229 85.77229) (end 85.141991 87.022589) (width 0.2) (layer "B.Cu") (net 1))
 (segment (start 94.01229 85.77229) (end 94.01229 87.737139) (width 0.2) (layer "B.Cu") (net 1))
 (segment (start 107.691991 94.637274) (end 110.091991 97.037274) (width 0.2) (layer "B.Cu") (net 1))
 (segment (start 101.491991 94.637274) (end 107.691991 94.637274) (width 0.2) (layer "B.Cu") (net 1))
 (segment (start 85.141991 87.022589) (end 85.141991 92.427274) (width 0.2) (layer "B.Cu") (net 1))
 (segment (start 86.396933 85.824752) (end 87.546933 84.674752) (width 0.2) (layer "B.Cu") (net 1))
 (segment (start 85.141991 92.427274) (end 86.291991 93.577274) (width 0.2) (layer "B.Cu") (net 1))
 (segment (start 92.866933 84.674752) (end 94.016933 85.824752) (width 0.2) (layer "B.Cu") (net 1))
 (segment (start 87.546933 84.674752) (end 92.866933 84.674752) (width 0.2) (layer "B.Cu") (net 1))
 (segment (start 95.291991 92.312274) (end 96.941991 92.312274) (width 0.2) (layer "F.Cu") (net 33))
 (segment (start 96.941991 92.312274) (end 97.666991 93.037274) (width 0.2) (layer "F.Cu") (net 33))
 (segment (start 91.791991 99.09092) (end 91.77998 99.078909) (width 0.2) (layer "F.Cu") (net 34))
 (segment (start 91.791991 99.983627) (end 91.791991 99.09092) (width 0.2) (layer "F.Cu") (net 34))
 (segment (start 88.291991 91.387274) (end 89.46289 91.387274) (width 0.2) (layer "F.Cu") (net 32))
 (segment (start 89.46289 91.387274) (end 89.592463 91.516847) (width 0.2) (layer "F.Cu") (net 32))
 (segment (start 104.591991 90.312274) (end 104.316991 90.037274) (width 0.2) (layer "F.Cu") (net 29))
 (segment (start 88.871991 104.037274) (end 88.871991 98.697274) (width 0.2) (layer "F.Cu") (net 29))
 (segment (start 92.371991 90.037274) (end 86.291991 96.117274) (width 0.2) (layer "F.Cu") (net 29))
 (segment (start 88.871991 98.697274) (end 86.291991 96.117274) (width 0.2) (layer "F.Cu") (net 29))
 (segment (start 104.591991 90.737274) (end 104.591991 90.312274) (width 0.2) (layer "F.Cu") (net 29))
 (segment (start 104.316991 90.037274) (end 92.371991 90.037274) (width 0.2) (layer "F.Cu") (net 29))
 (segment (start 111.751991 101.537274) (end 107.791991 101.537274) (width 0.2) (layer "F.Cu") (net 22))
 (segment (start 106.191991 99.937274) (end 107.791991 101.537274) (width 0.2) (layer "F.Cu") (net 22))
 (segment (start 114.251991 104.037274) (end 111.751991 101.537274) (width 0.2) (layer "F.Cu") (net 22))
 (segment (start 106.191991 99.337274) (end 106.191991 99.937274) (width 0.2) (layer "F.Cu") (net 22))
 (segment (start 99.991991 92.512274) (end 101.766991 90.737274) (width 0.2) (layer "F.Cu") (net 31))
 (segment (start 99.991991 100.537274) (end 99.991991 92.512274) (width 0.2) (layer "F.Cu") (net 31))
 (segment (start 101.766991 90.737274) (end 102.991991 90.737274) (width 0.2) (layer "F.Cu") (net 31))
 (segment (start 96.491991 104.037274) (end 99.991991 100.537274) (width 0.2) (layer "F.Cu") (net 31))
 (segment (start 102.991991 102.937274) (end 102.991991 99.337274) (width 0.2) (layer "F.Cu") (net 18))
 (segment (start 104.091991 104.037274) (end 102.991991 102.937274) (width 0.2) (layer "F.Cu") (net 18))
 (segment (start 91.506256 91.751539) (end 94.791991 95.037274) (width 0.2) (layer "F.Cu") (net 3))
 (segment (start 104.891991 89.637274) (end 105.391991 90.137274) (width 0.2) (layer "F.Cu") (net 3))
 (segment (start 91.47229 85.77229) (end 95.337274 89.637274) (width 0.2) (layer "F.Cu") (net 3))
 (segment (start 94.791991 95.037274) (end 94.791991 96.037274) (width 0.2) (layer "F.Cu") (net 3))
 (segment (start 95.337274 89.637274) (end 104.891991 89.637274) (width 0.2) (layer "F.Cu") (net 3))
 (segment (start 105.391991 90.137274) (end 105.391991 90.737274) (width 0.2) (layer "F.Cu") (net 3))
 (segment (start 97.691991 94.537274) (end 96.466991 95.762274) (width 0.2) (layer "F.Cu") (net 3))
 (segment (start 96.466991 95.762274) (end 95.291991 95.762274) (width 0.2) (layer "F.Cu") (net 3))
 (via (at 91.506256 91.751539) (size 0.55) (drill 0.15) (layers "F.Cu" "B.Cu") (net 3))
 (via (at 94.791991 96.037274) (size 0.55) (drill 0.15) (layers "F.Cu" "B.Cu") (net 3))
 (segment (start 91.506256 91.751539) (end 91.47229 91.717573) (width 0.2) (layer "B.Cu") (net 3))
 (segment (start 88.571991 101.197274) (end 91.411991 104.037274) (width 0.2) (layer "B.Cu") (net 3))
 (segment (start 89.631991 101.197274) (end 94.791991 96.037274) (width 0.2) (layer "B.Cu") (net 3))
 (segment (start 91.47229 91.717573) (end 91.47229 85.77229) (width 0.2) (layer "B.Cu") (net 3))
 (segment (start 88.571991 101.197274) (end 89.631991 101.197274) (width 0.2) (layer "B.Cu") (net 3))
 (segment (start 86.291991 101.197274) (end 88.571991 101.197274) (width 0.2) (layer "B.Cu") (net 3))
 (via (at 103.791991 90.737274) (size 0.55) (drill 0.15) (layers "F.Cu" "B.Cu") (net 30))
 (segment (start 86.291991 98.657274) (end 85.141991 99.807274) (width 0.2) (layer "B.Cu") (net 30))
 (segment (start 103.791991 90.737274) (end 103.591991 90.737274) (width 0.2) (layer "B.Cu") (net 30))
 (segment (start 93.411991 91.537274) (end 102.791991 91.537274) (width 0.2) (layer "B.Cu") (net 30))
 (segment (start 103.591991 90.737274) (end 102.791991 91.537274) (width 0.2) (layer "B.Cu") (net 30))
 (segment (start 85.141991 99.807274) (end 85.141991 102.847274) (width 0.2) (layer "B.Cu") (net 30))
 (segment (start 85.141991 102.847274) (end 86.331991 104.037274) (width 0.2) (layer "B.Cu") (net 30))
 (segment (start 86.291991 98.657274) (end 93.411991 91.537274) (width 0.2) (layer "B.Cu") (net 30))
 (segment (start 105.391991 99.70296) (end 105.391991 99.337274) (width 0.2) (layer "F.Cu") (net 21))
 (segment (start 111.711991 104.037274) (end 109.611991 101.937274) (width 0.2) (layer "F.Cu") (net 21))
 (segment (start 107.626305 101.937274) (end 105.391991 99.70296) (width 0.2) (layer "F.Cu") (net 21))
 (segment (start 109.611991 101.937274) (end 107.626305 101.937274) (width 0.2) (layer "F.Cu") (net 21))
 (segment (start 101.066991 93.037274) (end 100.791991 93.312274) (width 0.2) (layer "F.Cu") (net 13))
 (segment (start 100.791991 93.312274) (end 100.791991 103.277274) (width 0.2) (layer "F.Cu") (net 13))
 (segment (start 100.791991 103.277274) (end 101.551991 104.037274) (width 0.2) (layer "F.Cu") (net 13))
 (segment (start 101.491991 93.037274) (end 101.066991 93.037274) (width 0.2) (layer "F.Cu") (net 13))
 (segment (start 109.171991 104.037274) (end 108.691991 104.037274) (width 0.2) (layer "F.Cu") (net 20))
 (segment (start 108.691991 104.037274) (end 104.591991 99.937274) (width 0.2) (layer "F.Cu") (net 20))
 (segment (start 104.591991 99.937274) (end 104.591991 99.337274) (width 0.2) (layer "F.Cu") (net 20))
 (segment (start 100.391991 92.737274) (end 100.891991 92.237274) (width 0.2) (layer "F.Cu") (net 12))
 (segment (start 100.891991 92.237274) (end 101.491991 92.237274) (width 0.2) (layer "F.Cu") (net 12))
 (segment (start 99.031991 104.037274) (end 100.391991 102.677274) (width 0.2) (layer "F.Cu") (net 12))
 (segment (start 100.391991 102.677274) (end 100.391991 92.737274) (width 0.2) (layer "F.Cu") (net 12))
 (segment (start 103.791991 101.197274) (end 103.791991 99.337274) (width 0.2) (layer "F.Cu") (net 19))
 (segment (start 106.631991 104.037274) (end 103.791991 101.197274) (width 0.2) (layer "F.Cu") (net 19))
 (segment (start 110.893304 100.537274) (end 107.791991 100.537274) (width 0.2) (layer "F.Cu") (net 11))
 (segment (start 106.991991 99.737274) (end 106.991991 99.337274) (width 0.2) (layer "F.Cu") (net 11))
 (segment (start 114.31229 85.77229) (end 114.31229 97.118288) (width 0.2) (layer "F.Cu") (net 11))
 (segment (start 107.791991 100.537274) (end 106.991991 99.737274) (width 0.2) (layer "F.Cu") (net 11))
 (segment (start 114.31229 97.118288) (end 110.893304 100.537274) (width 0.2) (layer "F.Cu") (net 11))
 (segment (start 112.42771 91.50771) (end 112.42771 97.305811) (width 0.2) (layer "F.Cu") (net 8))
 (segment (start 106.69229 85.77229) (end 112.42771 91.50771) (width 0.2) (layer "F.Cu") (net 8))
 (segment (start 111.896247 97.837274) (end 110.091991 97.837274) (width 0.2) (layer "F.Cu") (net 8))
 (segment (start 112.42771 97.305811) (end 111.896247 97.837274) (width 0.2) (layer "F.Cu") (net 8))
 (via (at 91.791991 98.037274) (size 0.55) (drill 0.15) (layers "F.Cu" "B.Cu") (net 8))
 (segment (start 106.69229 90.636975) (end 105.023252 92.306013) (width 0.2) (layer "B.Cu") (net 8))
 (segment (start 106.69229 85.77229) (end 106.69229 90.636975) (width 0.2) (layer "B.Cu") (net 8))
 (segment (start 105.023252 92.306013) (end 97.523252 92.306013) (width 0.2) (layer "B.Cu") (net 8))
 (segment (start 97.523252 92.306013) (end 91.791991 98.037274) (width 0.2) (layer "B.Cu") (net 8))
 (segment (start 108.591991 90.137274) (end 108.591991 90.737274) (width 0.2) (layer "F.Cu") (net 5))
 (segment (start 107.291991 88.837274) (end 108.591991 90.137274) (width 0.2) (layer "F.Cu") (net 5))
 (segment (start 102.157274 88.837274) (end 107.291991 88.837274) (width 0.2) (layer "F.Cu") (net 5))
 (segment (start 99.09229 85.77229) (end 102.157274 88.837274) (width 0.2) (layer "F.Cu") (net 5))
 (segment (start 96.55229 85.77229) (end 100.017274 89.237274) (width 0.2) (layer "F.Cu") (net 4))
 (segment (start 100.017274 89.237274) (end 106.891991 89.237274) (width 0.2) (layer "F.Cu") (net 4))
 (segment (start 107.791991 90.137274) (end 107.791991 90.737274) (width 0.2) (layer "F.Cu") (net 4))
 (segment (start 106.891991 89.237274) (end 107.791991 90.137274) (width 0.2) (layer "F.Cu") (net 4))
 (segment (start 110.961933 99.337274) (end 108.591991 99.337274) (width 0.2) (layer "F.Cu") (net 9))
 (segment (start 109.23229 85.77229) (end 112.82771 89.36771) (width 0.2) (layer "F.Cu") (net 9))
 (segment (start 112.82771 89.36771) (end 112.82771 97.471497) (width 0.2) (layer "F.Cu") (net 9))
 (segment (start 112.82771 97.471497) (end 110.961933 99.337274) (width 0.2) (layer "F.Cu") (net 9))
 (segment (start 113.22771 87.22771) (end 111.77229 85.77229) (width 0.2) (layer "F.Cu") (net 10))
 (segment (start 107.791991 99.337274) (end 107.791991 99.762274) (width 0.2) (layer "F.Cu") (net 10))
 (segment (start 108.066991 100.037274) (end 110.827619 100.037274) (width 0.2) (layer "F.Cu") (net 10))
 (segment (start 107.791991 99.762274) (end 108.066991 100.037274) (width 0.2) (layer "F.Cu") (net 10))
 (segment (start 113.22771 97.637183) (end 113.22771 87.22771) (width 0.2) (layer "F.Cu") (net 10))
 (segment (start 110.827619 100.037274) (end 113.22771 97.637183) (width 0.2) (layer "F.Cu") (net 10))
 (segment (start 110.091991 91.071588) (end 110.091991 92.237274) (width 0.2) (layer "F.Cu") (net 6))
 (segment (start 107.457677 88.437274) (end 110.091991 91.071588) (width 0.2) (layer "F.Cu") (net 6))
 (segment (start 104.277274 88.437274) (end 107.457677 88.437274) (width 0.2) (layer "F.Cu") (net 6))
 (segment (start 101.61229 85.77229) (end 104.277274 88.437274) (width 0.2) (layer "F.Cu") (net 6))
 (segment (start 104.15229 85.77229) (end 106.417274 88.037274) (width 0.2) (layer "F.Cu") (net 7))
 (segment (start 110.791991 92.937274) (end 110.691991 93.037274) (width 0.2) (layer "F.Cu") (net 7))
 (segment (start 110.691991 93.037274) (end 110.091991 93.037274) (width 0.2) (layer "F.Cu") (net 7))
 (segment (start 110.791991 91.205902) (end 110.791991 92.937274) (width 0.2) (layer "F.Cu") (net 7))
 (segment (start 107.623363 88.037274) (end 110.791991 91.205902) (width 0.2) (layer "F.Cu") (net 7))
 (segment (start 106.417274 88.037274) (end 107.623363 88.037274) (width 0.2) (layer "F.Cu") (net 7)))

